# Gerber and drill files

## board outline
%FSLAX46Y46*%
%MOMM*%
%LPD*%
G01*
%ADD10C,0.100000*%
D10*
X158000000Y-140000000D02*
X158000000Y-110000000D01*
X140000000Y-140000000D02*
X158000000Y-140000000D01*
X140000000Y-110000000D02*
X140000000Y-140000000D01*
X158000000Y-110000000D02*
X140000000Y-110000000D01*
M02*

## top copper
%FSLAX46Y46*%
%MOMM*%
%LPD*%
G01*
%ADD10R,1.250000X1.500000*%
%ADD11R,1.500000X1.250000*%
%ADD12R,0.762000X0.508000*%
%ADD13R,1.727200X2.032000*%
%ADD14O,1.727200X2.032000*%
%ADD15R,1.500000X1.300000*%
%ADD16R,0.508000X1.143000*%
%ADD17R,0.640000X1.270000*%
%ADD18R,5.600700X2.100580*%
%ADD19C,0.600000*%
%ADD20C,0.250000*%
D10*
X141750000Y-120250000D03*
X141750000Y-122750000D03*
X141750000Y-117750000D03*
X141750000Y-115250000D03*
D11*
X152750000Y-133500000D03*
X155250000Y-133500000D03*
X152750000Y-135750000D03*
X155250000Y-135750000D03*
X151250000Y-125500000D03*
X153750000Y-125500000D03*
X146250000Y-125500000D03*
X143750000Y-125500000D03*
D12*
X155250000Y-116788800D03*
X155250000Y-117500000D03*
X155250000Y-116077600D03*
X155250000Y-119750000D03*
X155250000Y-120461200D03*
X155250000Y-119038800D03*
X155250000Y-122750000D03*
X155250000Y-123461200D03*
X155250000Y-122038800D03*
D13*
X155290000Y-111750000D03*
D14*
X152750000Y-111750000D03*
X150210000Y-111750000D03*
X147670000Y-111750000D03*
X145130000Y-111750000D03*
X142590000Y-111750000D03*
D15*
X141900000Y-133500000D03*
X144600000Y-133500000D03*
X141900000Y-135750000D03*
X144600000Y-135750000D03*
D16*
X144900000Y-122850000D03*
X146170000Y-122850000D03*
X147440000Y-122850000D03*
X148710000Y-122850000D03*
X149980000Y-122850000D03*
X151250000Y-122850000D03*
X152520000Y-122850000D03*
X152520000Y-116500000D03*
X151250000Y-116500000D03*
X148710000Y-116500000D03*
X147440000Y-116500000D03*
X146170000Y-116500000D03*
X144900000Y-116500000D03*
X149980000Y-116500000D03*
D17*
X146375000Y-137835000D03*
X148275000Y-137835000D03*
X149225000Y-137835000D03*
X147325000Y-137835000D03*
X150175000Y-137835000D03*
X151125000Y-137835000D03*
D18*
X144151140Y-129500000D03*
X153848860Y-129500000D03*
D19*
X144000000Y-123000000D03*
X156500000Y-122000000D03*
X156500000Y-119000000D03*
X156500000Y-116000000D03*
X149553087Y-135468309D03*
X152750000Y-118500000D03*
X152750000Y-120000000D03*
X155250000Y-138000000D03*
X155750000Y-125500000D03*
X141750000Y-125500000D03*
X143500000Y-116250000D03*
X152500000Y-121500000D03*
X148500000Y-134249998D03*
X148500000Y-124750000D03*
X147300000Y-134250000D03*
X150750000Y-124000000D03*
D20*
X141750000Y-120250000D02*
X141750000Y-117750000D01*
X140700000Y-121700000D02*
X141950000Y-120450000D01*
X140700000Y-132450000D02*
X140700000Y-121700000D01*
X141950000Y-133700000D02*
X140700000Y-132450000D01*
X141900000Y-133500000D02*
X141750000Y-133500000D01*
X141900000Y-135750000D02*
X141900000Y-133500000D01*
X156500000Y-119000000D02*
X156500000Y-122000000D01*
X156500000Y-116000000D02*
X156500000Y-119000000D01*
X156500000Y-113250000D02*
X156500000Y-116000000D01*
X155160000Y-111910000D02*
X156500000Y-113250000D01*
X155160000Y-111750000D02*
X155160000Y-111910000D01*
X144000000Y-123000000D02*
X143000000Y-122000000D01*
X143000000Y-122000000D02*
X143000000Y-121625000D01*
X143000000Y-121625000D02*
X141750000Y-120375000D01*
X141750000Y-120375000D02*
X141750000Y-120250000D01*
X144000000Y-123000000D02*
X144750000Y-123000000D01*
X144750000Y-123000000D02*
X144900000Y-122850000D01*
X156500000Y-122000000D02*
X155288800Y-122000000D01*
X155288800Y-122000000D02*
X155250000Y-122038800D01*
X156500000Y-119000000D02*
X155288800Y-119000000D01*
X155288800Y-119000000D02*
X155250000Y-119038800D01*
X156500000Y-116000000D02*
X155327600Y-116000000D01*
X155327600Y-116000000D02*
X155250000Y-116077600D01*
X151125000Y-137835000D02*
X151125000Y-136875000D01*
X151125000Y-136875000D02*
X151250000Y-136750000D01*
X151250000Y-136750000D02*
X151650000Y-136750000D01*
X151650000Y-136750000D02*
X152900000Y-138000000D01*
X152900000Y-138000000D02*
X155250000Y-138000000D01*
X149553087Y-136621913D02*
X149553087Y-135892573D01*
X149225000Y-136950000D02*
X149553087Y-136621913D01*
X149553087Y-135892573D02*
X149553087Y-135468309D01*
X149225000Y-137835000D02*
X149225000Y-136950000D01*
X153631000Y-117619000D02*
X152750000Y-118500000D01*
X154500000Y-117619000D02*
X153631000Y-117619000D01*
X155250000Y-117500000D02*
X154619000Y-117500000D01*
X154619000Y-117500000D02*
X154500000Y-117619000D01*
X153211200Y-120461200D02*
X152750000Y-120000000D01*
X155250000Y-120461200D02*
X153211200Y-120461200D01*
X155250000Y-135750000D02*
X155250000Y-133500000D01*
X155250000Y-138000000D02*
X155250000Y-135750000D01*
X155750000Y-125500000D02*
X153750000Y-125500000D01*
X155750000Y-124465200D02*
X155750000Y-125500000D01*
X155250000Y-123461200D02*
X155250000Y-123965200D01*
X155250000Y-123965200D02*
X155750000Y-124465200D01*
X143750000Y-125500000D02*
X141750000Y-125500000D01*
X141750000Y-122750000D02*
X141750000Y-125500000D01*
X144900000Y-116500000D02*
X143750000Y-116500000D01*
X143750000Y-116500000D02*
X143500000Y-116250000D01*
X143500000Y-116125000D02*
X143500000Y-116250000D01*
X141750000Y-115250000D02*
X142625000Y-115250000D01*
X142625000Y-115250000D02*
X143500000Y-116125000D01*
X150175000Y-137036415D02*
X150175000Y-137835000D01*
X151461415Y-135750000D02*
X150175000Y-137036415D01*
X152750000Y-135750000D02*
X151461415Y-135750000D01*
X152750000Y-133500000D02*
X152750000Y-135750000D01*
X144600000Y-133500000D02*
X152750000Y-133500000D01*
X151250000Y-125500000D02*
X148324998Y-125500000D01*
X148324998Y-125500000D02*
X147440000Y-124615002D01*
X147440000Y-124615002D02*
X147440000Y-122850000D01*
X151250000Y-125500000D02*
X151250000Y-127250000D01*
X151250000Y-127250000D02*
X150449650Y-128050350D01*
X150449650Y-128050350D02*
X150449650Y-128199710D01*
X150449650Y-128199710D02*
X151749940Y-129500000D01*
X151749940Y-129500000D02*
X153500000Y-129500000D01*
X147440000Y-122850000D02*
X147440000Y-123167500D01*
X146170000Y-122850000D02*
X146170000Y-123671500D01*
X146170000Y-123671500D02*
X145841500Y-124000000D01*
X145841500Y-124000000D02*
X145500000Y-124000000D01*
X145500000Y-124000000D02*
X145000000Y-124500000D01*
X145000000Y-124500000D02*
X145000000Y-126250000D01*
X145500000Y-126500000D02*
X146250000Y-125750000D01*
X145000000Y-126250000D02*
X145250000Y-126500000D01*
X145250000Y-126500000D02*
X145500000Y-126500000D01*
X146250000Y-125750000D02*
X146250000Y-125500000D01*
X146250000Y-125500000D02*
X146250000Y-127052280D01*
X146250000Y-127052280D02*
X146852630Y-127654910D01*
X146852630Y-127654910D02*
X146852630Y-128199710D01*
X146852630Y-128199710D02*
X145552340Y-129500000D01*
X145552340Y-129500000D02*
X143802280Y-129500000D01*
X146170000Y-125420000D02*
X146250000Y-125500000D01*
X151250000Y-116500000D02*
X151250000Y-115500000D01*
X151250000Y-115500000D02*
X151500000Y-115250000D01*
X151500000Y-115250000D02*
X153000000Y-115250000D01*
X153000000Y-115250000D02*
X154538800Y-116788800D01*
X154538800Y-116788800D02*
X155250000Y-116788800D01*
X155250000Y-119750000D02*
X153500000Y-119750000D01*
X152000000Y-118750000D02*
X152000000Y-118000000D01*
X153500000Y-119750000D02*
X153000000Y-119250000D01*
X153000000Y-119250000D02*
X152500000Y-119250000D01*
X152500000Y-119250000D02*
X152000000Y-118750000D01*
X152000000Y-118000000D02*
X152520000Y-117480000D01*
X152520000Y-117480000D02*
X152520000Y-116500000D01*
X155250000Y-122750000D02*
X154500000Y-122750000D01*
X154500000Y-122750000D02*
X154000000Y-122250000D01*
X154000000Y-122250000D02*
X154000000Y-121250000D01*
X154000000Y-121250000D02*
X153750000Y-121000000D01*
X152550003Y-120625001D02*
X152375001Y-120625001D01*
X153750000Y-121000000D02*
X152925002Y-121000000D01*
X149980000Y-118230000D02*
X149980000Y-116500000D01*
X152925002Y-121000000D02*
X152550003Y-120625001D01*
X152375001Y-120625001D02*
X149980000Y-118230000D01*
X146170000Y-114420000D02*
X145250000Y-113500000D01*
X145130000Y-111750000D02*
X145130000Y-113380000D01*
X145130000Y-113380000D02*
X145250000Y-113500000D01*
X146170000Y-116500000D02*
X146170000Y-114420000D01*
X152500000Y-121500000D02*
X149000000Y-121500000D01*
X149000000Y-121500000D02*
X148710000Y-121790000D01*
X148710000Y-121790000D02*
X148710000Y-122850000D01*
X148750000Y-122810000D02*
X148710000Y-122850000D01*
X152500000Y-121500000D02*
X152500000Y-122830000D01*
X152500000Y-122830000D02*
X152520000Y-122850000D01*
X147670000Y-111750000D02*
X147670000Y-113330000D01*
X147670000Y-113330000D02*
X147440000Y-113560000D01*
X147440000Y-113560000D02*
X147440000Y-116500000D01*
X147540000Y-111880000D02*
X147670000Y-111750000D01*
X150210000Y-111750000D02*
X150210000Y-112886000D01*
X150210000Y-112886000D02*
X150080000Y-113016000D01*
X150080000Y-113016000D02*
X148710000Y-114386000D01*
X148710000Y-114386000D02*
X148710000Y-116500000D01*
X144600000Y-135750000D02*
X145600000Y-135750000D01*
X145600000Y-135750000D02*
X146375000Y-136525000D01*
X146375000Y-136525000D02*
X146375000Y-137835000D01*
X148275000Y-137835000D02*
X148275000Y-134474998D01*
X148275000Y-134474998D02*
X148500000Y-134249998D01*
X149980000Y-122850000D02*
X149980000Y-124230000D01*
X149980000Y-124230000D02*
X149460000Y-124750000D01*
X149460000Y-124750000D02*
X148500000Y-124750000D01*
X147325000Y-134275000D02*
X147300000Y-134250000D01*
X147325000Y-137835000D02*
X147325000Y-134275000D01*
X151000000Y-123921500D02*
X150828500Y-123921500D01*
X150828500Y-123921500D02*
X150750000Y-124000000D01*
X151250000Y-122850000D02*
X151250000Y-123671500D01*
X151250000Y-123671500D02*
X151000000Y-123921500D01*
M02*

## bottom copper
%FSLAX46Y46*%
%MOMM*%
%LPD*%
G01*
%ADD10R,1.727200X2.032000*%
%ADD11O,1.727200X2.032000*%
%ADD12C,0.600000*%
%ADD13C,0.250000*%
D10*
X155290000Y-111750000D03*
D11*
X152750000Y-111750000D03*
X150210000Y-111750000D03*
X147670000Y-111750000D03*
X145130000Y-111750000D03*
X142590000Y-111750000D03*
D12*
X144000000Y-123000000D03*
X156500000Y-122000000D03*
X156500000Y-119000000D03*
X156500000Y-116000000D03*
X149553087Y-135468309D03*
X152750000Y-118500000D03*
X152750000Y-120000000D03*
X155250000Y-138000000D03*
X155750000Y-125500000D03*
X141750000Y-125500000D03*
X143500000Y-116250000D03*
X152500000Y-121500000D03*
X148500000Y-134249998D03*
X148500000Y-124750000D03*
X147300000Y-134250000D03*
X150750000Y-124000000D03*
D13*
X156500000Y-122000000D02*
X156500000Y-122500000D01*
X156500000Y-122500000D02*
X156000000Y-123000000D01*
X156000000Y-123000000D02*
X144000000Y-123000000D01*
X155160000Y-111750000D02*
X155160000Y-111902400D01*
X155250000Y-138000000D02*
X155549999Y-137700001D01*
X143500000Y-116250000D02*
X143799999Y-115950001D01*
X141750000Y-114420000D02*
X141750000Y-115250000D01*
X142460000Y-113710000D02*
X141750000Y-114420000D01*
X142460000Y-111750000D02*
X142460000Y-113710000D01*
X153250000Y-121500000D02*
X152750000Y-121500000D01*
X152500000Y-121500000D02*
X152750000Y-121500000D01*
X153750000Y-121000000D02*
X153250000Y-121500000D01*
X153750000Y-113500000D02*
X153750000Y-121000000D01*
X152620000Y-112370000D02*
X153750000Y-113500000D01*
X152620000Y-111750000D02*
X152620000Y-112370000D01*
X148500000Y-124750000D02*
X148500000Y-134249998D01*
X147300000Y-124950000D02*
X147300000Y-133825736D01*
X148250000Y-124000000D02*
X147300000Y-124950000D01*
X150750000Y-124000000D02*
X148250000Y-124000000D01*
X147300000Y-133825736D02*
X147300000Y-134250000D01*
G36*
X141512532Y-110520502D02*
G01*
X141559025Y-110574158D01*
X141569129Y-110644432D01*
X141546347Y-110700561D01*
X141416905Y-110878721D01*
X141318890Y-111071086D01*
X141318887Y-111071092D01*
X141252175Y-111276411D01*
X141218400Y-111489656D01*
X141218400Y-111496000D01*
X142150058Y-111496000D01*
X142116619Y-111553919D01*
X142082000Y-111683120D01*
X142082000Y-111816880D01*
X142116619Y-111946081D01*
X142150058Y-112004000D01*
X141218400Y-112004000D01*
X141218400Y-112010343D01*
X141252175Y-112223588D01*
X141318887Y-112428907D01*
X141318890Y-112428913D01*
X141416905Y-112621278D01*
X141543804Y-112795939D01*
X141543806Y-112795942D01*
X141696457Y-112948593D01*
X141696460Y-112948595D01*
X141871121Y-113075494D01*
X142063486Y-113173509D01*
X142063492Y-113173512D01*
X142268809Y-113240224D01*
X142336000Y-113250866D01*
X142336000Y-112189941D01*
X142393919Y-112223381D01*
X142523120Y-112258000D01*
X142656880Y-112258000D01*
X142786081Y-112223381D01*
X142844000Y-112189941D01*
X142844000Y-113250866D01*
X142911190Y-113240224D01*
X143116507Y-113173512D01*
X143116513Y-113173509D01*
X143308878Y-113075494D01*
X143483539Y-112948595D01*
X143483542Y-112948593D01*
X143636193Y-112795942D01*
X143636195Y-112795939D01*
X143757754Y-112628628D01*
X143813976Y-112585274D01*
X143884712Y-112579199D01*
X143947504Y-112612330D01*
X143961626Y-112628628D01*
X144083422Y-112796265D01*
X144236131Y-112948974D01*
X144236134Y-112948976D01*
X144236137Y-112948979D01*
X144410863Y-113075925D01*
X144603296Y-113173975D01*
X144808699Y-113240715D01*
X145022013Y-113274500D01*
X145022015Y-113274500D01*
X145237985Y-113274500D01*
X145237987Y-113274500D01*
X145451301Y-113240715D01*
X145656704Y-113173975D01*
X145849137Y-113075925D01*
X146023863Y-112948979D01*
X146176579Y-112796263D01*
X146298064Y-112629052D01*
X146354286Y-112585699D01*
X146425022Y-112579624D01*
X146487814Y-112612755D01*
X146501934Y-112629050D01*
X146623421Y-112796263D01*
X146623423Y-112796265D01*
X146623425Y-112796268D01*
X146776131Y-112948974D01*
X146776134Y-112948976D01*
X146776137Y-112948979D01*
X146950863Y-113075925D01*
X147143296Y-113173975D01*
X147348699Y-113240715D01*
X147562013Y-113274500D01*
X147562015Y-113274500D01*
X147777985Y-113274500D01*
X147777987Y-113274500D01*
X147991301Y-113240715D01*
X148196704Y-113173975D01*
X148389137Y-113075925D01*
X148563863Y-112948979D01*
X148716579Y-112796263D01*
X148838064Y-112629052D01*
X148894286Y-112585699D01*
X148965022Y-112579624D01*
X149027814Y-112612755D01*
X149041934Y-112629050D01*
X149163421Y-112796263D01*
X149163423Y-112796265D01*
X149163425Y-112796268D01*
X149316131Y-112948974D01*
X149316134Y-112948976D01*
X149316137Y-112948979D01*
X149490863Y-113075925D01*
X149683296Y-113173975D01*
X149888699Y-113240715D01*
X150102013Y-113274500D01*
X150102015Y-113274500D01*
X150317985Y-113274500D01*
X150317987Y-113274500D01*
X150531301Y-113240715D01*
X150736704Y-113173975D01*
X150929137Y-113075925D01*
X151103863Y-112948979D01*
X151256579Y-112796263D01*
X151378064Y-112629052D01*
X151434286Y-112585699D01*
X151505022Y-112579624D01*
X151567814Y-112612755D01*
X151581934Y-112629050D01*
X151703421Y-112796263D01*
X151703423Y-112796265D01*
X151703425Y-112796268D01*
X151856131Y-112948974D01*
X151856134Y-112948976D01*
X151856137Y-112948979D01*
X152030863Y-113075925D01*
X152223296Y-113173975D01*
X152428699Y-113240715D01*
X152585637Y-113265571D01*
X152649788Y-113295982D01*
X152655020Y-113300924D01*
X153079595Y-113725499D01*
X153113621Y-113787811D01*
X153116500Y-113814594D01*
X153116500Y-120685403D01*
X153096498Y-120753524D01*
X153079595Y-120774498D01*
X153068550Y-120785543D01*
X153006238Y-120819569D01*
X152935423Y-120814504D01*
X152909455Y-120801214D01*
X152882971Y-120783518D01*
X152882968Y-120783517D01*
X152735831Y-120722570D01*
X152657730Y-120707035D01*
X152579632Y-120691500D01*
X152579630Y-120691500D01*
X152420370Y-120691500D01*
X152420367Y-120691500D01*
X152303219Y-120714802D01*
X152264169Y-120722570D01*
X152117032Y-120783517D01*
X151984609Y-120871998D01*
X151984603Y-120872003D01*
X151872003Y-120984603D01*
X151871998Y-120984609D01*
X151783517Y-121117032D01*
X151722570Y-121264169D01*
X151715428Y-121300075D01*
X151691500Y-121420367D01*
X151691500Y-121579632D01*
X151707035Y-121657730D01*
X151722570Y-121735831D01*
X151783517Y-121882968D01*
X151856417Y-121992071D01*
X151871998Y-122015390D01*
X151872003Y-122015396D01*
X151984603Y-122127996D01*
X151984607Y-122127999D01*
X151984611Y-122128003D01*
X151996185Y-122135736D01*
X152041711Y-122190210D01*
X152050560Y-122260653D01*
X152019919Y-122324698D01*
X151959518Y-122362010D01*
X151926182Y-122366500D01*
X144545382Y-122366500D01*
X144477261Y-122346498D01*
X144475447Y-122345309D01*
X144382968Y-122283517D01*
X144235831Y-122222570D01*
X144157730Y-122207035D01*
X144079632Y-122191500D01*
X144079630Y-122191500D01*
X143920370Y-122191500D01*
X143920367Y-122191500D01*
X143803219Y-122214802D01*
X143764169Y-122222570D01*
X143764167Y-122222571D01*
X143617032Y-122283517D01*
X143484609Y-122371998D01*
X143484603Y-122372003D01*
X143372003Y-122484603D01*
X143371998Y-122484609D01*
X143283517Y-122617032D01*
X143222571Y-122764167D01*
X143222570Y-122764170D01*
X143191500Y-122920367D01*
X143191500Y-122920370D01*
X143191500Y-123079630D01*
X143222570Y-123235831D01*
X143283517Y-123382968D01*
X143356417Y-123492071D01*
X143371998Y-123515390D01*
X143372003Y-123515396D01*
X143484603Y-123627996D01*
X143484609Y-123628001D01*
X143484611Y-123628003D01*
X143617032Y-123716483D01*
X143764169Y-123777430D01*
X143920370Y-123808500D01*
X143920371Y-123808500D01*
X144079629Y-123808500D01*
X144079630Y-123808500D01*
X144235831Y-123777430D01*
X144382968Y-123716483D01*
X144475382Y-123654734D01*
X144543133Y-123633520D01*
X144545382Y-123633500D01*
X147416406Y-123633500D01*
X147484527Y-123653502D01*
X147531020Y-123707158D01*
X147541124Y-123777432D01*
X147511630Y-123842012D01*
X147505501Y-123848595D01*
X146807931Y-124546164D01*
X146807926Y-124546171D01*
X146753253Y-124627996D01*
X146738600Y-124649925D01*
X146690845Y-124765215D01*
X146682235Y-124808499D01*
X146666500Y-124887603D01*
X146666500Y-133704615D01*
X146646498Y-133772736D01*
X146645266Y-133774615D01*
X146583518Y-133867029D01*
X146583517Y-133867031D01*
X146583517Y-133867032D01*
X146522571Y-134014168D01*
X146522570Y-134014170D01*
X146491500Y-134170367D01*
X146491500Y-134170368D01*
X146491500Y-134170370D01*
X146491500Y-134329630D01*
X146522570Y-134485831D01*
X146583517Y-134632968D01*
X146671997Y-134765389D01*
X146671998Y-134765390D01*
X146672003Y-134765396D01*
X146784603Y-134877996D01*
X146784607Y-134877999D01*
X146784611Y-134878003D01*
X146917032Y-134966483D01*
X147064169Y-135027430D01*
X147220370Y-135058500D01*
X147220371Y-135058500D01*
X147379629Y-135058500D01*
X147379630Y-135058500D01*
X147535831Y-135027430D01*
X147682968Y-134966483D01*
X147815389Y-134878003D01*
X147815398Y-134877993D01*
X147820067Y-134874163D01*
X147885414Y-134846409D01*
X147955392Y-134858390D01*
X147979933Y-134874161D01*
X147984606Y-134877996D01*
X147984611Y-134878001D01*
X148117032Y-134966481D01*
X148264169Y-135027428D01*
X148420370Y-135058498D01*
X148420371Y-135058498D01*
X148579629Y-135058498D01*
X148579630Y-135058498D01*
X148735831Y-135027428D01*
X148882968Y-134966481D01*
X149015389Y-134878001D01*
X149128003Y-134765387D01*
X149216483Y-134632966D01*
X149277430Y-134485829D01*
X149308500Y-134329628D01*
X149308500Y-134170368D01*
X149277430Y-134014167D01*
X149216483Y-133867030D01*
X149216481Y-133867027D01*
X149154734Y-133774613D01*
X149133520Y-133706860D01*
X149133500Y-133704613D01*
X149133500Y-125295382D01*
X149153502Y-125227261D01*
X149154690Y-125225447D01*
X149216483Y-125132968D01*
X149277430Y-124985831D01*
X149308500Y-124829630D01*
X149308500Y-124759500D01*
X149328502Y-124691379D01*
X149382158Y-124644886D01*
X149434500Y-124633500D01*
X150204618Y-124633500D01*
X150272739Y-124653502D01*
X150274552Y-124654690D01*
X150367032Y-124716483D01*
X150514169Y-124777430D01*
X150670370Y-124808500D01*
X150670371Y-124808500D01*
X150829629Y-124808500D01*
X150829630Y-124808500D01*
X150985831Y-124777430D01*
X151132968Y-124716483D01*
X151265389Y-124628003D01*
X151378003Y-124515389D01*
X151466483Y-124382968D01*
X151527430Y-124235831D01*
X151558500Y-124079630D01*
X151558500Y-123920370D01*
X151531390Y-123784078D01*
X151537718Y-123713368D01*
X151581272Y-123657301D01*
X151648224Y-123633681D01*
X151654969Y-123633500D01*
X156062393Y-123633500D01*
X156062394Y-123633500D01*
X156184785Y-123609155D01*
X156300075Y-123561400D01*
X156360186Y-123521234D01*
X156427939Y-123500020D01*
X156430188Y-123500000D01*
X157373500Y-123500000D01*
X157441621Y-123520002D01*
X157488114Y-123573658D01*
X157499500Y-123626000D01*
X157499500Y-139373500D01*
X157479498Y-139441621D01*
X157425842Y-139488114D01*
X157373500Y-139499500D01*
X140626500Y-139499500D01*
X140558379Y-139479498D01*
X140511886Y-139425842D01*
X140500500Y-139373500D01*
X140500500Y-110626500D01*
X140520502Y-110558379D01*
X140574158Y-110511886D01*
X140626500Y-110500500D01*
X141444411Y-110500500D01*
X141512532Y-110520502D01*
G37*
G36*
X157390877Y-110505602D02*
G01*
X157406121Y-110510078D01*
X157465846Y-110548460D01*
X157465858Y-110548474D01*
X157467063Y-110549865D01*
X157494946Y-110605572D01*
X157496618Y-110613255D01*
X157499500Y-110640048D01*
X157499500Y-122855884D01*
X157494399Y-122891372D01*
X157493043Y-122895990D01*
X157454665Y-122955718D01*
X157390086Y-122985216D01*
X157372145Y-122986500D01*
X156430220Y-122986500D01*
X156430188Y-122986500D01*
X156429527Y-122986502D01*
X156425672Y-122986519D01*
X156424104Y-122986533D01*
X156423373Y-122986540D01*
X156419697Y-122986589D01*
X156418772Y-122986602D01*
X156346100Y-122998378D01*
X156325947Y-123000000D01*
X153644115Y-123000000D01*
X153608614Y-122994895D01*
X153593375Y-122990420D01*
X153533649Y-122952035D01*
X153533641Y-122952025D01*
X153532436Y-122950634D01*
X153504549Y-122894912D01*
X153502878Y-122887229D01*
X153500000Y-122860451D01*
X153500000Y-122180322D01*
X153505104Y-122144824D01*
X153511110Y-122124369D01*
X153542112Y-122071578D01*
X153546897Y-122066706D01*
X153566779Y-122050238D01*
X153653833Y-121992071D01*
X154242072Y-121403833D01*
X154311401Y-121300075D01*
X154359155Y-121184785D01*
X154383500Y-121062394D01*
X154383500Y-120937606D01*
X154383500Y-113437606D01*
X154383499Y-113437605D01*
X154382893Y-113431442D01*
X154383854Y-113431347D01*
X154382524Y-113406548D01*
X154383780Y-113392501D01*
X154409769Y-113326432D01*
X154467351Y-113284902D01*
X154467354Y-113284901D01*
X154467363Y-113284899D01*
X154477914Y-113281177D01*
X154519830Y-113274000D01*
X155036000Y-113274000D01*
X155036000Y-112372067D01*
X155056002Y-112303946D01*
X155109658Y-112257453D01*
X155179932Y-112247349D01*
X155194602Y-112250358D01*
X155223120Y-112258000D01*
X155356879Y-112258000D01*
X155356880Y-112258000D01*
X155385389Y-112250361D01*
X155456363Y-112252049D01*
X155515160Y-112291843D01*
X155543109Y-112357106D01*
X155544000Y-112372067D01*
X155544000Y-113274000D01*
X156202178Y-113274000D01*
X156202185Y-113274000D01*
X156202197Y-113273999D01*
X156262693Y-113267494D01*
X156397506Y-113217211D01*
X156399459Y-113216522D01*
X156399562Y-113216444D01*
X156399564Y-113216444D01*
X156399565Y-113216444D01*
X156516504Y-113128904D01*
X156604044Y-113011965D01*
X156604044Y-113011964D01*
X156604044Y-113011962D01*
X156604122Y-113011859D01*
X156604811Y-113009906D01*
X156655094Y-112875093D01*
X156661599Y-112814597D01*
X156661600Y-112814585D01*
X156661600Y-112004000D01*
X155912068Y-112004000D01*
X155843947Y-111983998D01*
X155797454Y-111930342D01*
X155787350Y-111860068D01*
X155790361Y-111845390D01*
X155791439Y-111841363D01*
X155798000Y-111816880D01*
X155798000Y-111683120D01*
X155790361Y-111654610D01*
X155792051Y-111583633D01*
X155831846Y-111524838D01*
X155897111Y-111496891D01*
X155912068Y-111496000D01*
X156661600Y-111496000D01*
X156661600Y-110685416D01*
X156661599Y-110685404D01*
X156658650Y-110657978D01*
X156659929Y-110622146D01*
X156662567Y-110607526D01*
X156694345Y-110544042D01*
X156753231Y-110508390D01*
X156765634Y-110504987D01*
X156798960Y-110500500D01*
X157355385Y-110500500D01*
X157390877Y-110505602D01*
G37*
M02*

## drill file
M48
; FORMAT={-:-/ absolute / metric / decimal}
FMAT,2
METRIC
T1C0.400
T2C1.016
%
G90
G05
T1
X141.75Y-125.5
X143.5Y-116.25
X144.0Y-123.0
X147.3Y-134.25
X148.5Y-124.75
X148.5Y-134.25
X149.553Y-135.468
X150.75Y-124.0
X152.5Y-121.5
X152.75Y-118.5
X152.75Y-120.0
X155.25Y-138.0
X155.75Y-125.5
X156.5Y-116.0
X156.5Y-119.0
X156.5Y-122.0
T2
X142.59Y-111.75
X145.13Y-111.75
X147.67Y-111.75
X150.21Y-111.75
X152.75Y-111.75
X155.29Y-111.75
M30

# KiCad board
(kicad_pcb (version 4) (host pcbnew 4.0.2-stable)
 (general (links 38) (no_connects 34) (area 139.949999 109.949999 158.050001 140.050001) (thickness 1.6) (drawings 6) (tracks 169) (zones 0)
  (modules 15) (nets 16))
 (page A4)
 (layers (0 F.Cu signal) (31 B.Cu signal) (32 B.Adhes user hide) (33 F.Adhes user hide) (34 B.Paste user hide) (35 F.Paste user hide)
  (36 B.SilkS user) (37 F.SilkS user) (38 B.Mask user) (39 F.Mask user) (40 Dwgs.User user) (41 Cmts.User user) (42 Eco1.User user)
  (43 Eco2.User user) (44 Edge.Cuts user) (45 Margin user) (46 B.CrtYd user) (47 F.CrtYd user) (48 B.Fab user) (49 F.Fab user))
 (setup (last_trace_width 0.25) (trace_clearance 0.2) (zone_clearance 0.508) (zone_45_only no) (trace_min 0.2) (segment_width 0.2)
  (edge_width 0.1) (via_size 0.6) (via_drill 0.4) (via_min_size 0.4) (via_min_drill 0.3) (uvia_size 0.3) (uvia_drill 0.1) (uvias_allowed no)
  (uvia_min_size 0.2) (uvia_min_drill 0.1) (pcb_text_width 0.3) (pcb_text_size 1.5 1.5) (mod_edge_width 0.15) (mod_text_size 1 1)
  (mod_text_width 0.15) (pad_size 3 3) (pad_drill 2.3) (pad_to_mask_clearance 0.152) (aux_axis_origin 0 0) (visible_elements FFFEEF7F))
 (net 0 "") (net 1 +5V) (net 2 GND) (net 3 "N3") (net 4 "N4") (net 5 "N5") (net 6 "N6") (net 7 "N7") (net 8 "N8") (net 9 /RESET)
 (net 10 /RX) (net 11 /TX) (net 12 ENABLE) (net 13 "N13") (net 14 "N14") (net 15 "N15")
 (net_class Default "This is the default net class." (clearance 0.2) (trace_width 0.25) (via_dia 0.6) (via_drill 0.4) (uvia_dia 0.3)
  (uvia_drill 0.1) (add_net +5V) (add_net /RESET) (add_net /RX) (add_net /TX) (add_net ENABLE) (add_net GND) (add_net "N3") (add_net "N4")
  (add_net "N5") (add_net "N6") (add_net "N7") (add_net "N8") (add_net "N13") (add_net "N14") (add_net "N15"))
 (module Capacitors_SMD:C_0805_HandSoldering (layer F.Cu) (at 141.75 121.5 270)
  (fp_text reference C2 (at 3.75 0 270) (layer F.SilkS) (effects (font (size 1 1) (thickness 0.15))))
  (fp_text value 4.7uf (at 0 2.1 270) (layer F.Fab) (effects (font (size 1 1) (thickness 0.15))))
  (pad 1 smd rect (at -1.25 0 270) (size 1.5 1.25) (layers F.Cu F.Paste F.Mask) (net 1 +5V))
  (pad 2 smd rect (at 1.25 0 270) (size 1.5 1.25) (layers F.Cu F.Paste F.Mask) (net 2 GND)))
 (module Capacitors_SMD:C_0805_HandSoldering (layer F.Cu) (at 141.75 116.5 90)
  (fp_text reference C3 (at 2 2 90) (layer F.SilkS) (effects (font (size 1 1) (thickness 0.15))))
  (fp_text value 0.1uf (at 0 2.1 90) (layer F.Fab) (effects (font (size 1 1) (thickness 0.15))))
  (pad 1 smd rect (at -1.25 0 90) (size 1.5 1.25) (layers F.Cu F.Paste F.Mask) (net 1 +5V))
  (pad 2 smd rect (at 1.25 0 90) (size 1.5 1.25) (layers F.Cu F.Paste F.Mask) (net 2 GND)))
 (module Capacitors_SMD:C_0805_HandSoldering (layer F.Cu) (at 154 133.5)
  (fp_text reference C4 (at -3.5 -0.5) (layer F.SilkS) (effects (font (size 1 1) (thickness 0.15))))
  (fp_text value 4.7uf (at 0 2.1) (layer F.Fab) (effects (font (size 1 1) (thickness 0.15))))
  (pad 1 smd rect (at -1.25 0) (size 1.5 1.25) (layers F.Cu F.Paste F.Mask) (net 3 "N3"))
  (pad 2 smd rect (at 1.25 0) (size 1.5 1.25) (layers F.Cu F.Paste F.Mask) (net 2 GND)))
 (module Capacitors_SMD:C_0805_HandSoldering (layer F.Cu) (at 154 135.75)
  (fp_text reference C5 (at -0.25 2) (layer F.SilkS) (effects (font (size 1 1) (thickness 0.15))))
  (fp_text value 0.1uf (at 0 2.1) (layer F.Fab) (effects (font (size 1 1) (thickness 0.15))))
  (pad 1 smd rect (at -1.25 0) (size 1.5 1.25) (layers F.Cu F.Paste F.Mask) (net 3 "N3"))
  (pad 2 smd rect (at 1.25 0) (size 1.5 1.25) (layers F.Cu F.Paste F.Mask) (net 2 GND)))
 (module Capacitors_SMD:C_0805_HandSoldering (layer F.Cu) (at 152.5 125.5)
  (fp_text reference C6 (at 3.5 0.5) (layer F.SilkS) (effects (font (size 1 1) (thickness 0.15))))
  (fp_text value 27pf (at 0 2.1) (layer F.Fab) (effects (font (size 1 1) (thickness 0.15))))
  (pad 1 smd rect (at -1.25 0) (size 1.5 1.25) (layers F.Cu F.Paste F.Mask) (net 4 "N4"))
  (pad 2 smd rect (at 1.25 0) (size 1.5 1.25) (layers F.Cu F.Paste F.Mask) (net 2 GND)))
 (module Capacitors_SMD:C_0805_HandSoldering (layer F.Cu) (at 145 125.5 180)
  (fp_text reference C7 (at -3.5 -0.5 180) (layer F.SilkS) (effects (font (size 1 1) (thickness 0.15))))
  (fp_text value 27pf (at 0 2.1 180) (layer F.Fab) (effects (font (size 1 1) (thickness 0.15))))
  (pad 1 smd rect (at -1.25 0 180) (size 1.5 1.25) (layers F.Cu F.Paste F.Mask) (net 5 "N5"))
  (pad 2 smd rect (at 1.25 0 180) (size 1.5 1.25) (layers F.Cu F.Paste F.Mask) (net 2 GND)))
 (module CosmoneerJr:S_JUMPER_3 (layer F.Cu) (at 155.25 116.7888 90)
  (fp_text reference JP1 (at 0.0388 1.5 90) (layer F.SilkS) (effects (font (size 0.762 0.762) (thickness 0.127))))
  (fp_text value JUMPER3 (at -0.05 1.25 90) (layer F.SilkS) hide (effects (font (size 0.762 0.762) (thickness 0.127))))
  (pad 2 smd rect (at 0 0 90) (size 0.508 0.762) (layers F.Cu F.Paste F.Mask) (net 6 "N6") (clearance 0.2032))
  (pad 1 smd rect (at -0.7112 0 90) (size 0.508 0.762) (layers F.Cu F.Paste F.Mask) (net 2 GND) (clearance 0.2032))
  (pad 3 smd rect (at 0.7112 0 90) (size 0.508 0.762) (layers F.Cu F.Paste F.Mask) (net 1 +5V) (clearance 0.2032)))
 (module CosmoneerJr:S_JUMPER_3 (layer F.Cu) (at 155.25 119.75 90)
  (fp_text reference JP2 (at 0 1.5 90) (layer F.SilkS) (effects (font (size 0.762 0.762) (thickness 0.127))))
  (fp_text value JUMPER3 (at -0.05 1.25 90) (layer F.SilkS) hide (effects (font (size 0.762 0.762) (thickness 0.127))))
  (pad 2 smd rect (at 0 0 90) (size 0.508 0.762) (layers F.Cu F.Paste F.Mask) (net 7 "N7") (clearance 0.2032))
  (pad 1 smd rect (at -0.7112 0 90) (size 0.508 0.762) (layers F.Cu F.Paste F.Mask) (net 2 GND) (clearance 0.2032))
  (pad 3 smd rect (at 0.7112 0 90) (size 0.508 0.762) (layers F.Cu F.Paste F.Mask) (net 1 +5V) (clearance 0.2032)))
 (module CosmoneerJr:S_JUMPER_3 (layer F.Cu) (at 155.25 122.75 90)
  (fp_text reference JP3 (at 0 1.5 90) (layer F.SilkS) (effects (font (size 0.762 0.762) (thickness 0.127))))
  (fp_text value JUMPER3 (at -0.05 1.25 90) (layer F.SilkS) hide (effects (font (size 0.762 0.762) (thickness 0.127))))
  (pad 2 smd rect (at 0 0 90) (size 0.508 0.762) (layers F.Cu F.Paste F.Mask) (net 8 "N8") (clearance 0.2032))
  (pad 1 smd rect (at -0.7112 0 90) (size 0.508 0.762) (layers F.Cu F.Paste F.Mask) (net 2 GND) (clearance 0.2032))
  (pad 3 smd rect (at 0.7112 0 90) (size 0.508 0.762) (layers F.Cu F.Paste F.Mask) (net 1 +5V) (clearance 0.2032)))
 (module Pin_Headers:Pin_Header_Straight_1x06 (layer F.Cu) (at 155.29 111.75 270)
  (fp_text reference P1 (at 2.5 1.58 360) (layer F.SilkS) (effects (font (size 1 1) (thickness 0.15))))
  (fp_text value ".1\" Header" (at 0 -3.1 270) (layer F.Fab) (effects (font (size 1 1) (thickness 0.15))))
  (pad 1 thru_hole rect (at 0 0 270) (size 2.032 1.7272) (drill 1.016) (layers *.Cu *.Mask F.SilkS) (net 1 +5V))
  (pad 2 thru_hole oval (at 0 2.54 270) (size 2.032 1.7272) (drill 1.016) (layers *.Cu *.Mask F.SilkS) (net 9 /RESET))
  (pad 3 thru_hole oval (at 0 5.08 270) (size 2.032 1.7272) (drill 1.016) (layers *.Cu *.Mask F.SilkS) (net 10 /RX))
  (pad 4 thru_hole oval (at 0 7.62 270) (size 2.032 1.7272) (drill 1.016) (layers *.Cu *.Mask F.SilkS) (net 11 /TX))
  (pad 5 thru_hole oval (at 0 10.16 270) (size 2.032 1.7272) (drill 1.016) (layers *.Cu *.Mask F.SilkS) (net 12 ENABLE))
  (pad 6 thru_hole oval (at 0 12.7 270) (size 2.032 1.7272) (drill 1.016) (layers *.Cu *.Mask F.SilkS) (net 2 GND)))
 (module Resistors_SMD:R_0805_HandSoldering (layer F.Cu) (at 143.25 133.5)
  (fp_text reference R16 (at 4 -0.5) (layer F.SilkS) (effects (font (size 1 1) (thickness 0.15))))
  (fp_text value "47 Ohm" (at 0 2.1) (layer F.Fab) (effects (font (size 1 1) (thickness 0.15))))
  (pad 1 smd rect (at -1.35 0) (size 1.5 1.3) (layers F.Cu F.Paste F.Mask) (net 1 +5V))
  (pad 2 smd rect (at 1.35 0) (size 1.5 1.3) (layers F.Cu F.Paste F.Mask) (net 3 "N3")))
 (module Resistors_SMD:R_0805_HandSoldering (layer F.Cu) (at 143.25 135.75)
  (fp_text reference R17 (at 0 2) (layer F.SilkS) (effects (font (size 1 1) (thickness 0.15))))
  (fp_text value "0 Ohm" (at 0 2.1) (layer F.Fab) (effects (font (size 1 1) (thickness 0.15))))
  (pad 1 smd rect (at -1.35 0) (size 1.5 1.3) (layers F.Cu F.Paste F.Mask) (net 1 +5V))
  (pad 2 smd rect (at 1.35 0) (size 1.5 1.3) (layers F.Cu F.Paste F.Mask) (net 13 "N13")))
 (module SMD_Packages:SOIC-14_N (layer F.Cu) (at 148.71 119.548)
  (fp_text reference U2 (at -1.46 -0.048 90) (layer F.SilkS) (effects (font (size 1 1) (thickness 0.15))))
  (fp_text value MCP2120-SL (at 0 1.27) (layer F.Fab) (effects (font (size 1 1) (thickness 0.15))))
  (pad 1 smd rect (at -3.81 3.302) (size 0.508 1.143) (layers F.Cu F.Paste F.Mask) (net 1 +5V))
  (pad 2 smd rect (at -2.54 3.302) (size 0.508 1.143) (layers F.Cu F.Paste F.Mask) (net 5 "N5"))
  (pad 3 smd rect (at -1.27 3.302) (size 0.508 1.143) (layers F.Cu F.Paste F.Mask) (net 4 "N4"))
  (pad 4 smd rect (at 0 3.302) (size 0.508 1.143) (layers F.Cu F.Paste F.Mask) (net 9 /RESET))
  (pad 5 smd rect (at 1.27 3.302) (size 0.508 1.143) (layers F.Cu F.Paste F.Mask) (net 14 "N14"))
  (pad 6 smd rect (at 2.54 3.302) (size 0.508 1.143) (layers F.Cu F.Paste F.Mask) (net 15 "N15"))
  (pad 7 smd rect (at 3.81 3.302) (size 0.508 1.143) (layers F.Cu F.Paste F.Mask) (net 9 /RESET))
  (pad 8 smd rect (at 3.81 -3.048) (size 0.508 1.143) (layers F.Cu F.Paste F.Mask) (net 7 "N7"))
  (pad 9 smd rect (at 2.54 -3.048) (size 0.508 1.143) (layers F.Cu F.Paste F.Mask) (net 6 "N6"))
  (pad 11 smd rect (at 0 -3.048) (size 0.508 1.143) (layers F.Cu F.Paste F.Mask) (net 10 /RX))
  (pad 12 smd rect (at -1.27 -3.048) (size 0.508 1.143) (layers F.Cu F.Paste F.Mask) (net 11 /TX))
  (pad 13 smd rect (at -2.54 -3.048) (size 0.508 1.143) (layers F.Cu F.Paste F.Mask) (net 12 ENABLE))
  (pad 14 smd rect (at -3.81 -3.048) (size 0.508 1.143) (layers F.Cu F.Paste F.Mask) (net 2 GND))
  (pad 10 smd rect (at 1.27 -3.048) (size 0.508 1.143) (layers F.Cu F.Paste F.Mask) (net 8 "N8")))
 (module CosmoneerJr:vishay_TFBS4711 (layer F.Cu) (at 148.75 138.5)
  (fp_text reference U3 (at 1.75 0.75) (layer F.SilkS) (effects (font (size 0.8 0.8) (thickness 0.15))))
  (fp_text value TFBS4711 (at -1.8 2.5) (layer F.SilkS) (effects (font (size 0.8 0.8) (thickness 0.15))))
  (pad 1 smd rect (at -2.375 -0.665) (size 0.64 1.27) (layers F.Cu F.Paste F.Mask) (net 13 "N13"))
  (pad 3 smd rect (at -0.475 -0.665) (size 0.64 1.27) (layers F.Cu F.Paste F.Mask) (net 14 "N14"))
  (pad 4 smd rect (at 0.475 -0.665) (size 0.64 1.27) (layers F.Cu F.Paste F.Mask) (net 2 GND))
  (pad 2 smd rect (at -1.425 -0.665) (size 0.64 1.27) (layers F.Cu F.Paste F.Mask) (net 15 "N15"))
  (pad 5 smd rect (at 1.425 -0.665) (size 0.64 1.27) (layers F.Cu F.Paste F.Mask) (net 3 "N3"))
  (pad 6 smd rect (at 2.375 -0.665) (size 0.64 1.27) (layers F.Cu F.Paste F.Mask) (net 2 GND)))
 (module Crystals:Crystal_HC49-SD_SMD (layer F.Cu) (at 149 129.5)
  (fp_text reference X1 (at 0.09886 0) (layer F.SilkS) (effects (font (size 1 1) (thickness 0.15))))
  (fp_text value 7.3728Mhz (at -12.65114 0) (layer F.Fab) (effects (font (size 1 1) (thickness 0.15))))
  (pad 1 smd rect (at -4.84886 0) (size 5.6007 2.10058) (layers F.Cu F.Paste F.Mask) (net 5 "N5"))
  (pad 2 smd rect (at 4.84886 0) (size 5.6007 2.10058) (layers F.Cu F.Paste F.Mask) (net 4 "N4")))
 (gr_line (start 158 140) (end 158 110) (layer Edge.Cuts) (width 0.1))
 (gr_line (start 140 140) (end 158 140) (layer Edge.Cuts) (width 0.1))
 (gr_line (start 140 110) (end 140 140) (layer Edge.Cuts) (width 0.1))
 (gr_line (start 158 110) (end 140 110) (layer Edge.Cuts) (width 0.1))
 (segment (start 141.75 120.25) (end 141.75 117.75) (width 0.25) (layer F.Cu) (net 1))
 (segment (start 140.7 121.7) (end 141.95 120.45) (width 0.25) (layer F.Cu) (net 1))
 (segment (start 140.7 132.45) (end 140.7 121.7) (width 0.25) (layer F.Cu) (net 1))
 (segment (start 141.95 133.7) (end 140.7 132.45) (width 0.25) (layer F.Cu) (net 1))
 (segment (start 141.9 133.5) (end 141.75 133.5) (width 0.25) (layer F.Cu) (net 1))
 (segment (start 141.9 135.75) (end 141.9 133.5) (width 0.25) (layer F.Cu) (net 1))
 (segment (start 156.5 119) (end 156.5 122) (width 0.25) (layer F.Cu) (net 1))
 (segment (start 156.5 116) (end 156.5 119) (width 0.25) (layer F.Cu) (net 1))
 (segment (start 156.5 113.25) (end 156.5 116) (width 0.25) (layer F.Cu) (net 1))
 (segment (start 155.16 111.91) (end 156.5 113.25) (width 0.25) (layer F.Cu) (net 1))
 (segment (start 155.16 111.75) (end 155.16 111.91) (width 0.25) (layer F.Cu) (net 1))
 (segment (start 144 123) (end 143 122) (width 0.25) (layer F.Cu) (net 1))
 (segment (start 143 122) (end 143 121.625) (width 0.25) (layer F.Cu) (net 1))
 (segment (start 143 121.625) (end 141.75 120.375) (width 0.25) (layer F.Cu) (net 1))
 (segment (start 141.75 120.375) (end 141.75 120.25) (width 0.25) (layer F.Cu) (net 1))
 (segment (start 144 123) (end 144.75 123) (width 0.25) (layer F.Cu) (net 1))
 (segment (start 144.75 123) (end 144.9 122.85) (width 0.25) (layer F.Cu) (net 1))
 (via (at 144 123) (size 0.6) (drill 0.4) (layers F.Cu B.Cu) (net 1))
 (segment (start 156.5 122) (end 156.5 122.5) (width 0.25) (layer B.Cu) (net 1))
 (segment (start 156.5 122.5) (end 156 123) (width 0.25) (layer B.Cu) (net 1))
 (segment (start 156 123) (end 144 123) (width 0.25) (layer B.Cu) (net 1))
 (segment (start 156.5 122) (end 155.2888 122) (width 0.25) (layer F.Cu) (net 1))
 (segment (start 155.2888 122) (end 155.25 122.0388) (width 0.25) (layer F.Cu) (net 1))
 (segment (start 156.5 119) (end 155.2888 119) (width 0.25) (layer F.Cu) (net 1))
 (segment (start 155.2888 119) (end 155.25 119.0388) (width 0.25) (layer F.Cu) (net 1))
 (via (at 156.5 122) (size 0.6) (drill 0.4) (layers F.Cu B.Cu) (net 1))
 (via (at 156.5 119) (size 0.6) (drill 0.4) (layers F.Cu B.Cu) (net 1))
 (segment (start 156.5 116) (end 155.3276 116) (width 0.25) (layer F.Cu) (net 1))
 (segment (start 155.3276 116) (end 155.25 116.0776) (width 0.25) (layer F.Cu) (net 1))
 (via (at 156.5 116) (size 0.6) (drill 0.4) (layers F.Cu B.Cu) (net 1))
 (segment (start 155.16 111.75) (end 155.16 111.9024) (width 0.25) (layer B.Cu) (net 1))
 (segment (start 151.125 137.835) (end 151.125 136.875) (width 0.25) (layer F.Cu) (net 2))
 (segment (start 151.125 136.875) (end 151.25 136.75) (width 0.25) (layer F.Cu) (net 2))
 (segment (start 151.25 136.75) (end 151.65 136.75) (width 0.25) (layer F.Cu) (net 2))
 (segment (start 151.65 136.75) (end 152.9 138) (width 0.25) (layer F.Cu) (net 2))
 (segment (start 152.9 138) (end 155.25 138) (width 0.25) (layer F.Cu) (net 2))
 (segment (start 149.553087 136.621913) (end 149.553087 135.892573) (width 0.25) (layer F.Cu) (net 2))
 (segment (start 149.225 136.95) (end 149.553087 136.621913) (width 0.25) (layer F.Cu) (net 2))
 (segment (start 149.553087 135.892573) (end 149.553087 135.468309) (width 0.25) (layer F.Cu) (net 2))
 (via (at 149.553087 135.468309) (size 0.6) (drill 0.4) (layers F.Cu B.Cu) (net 2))
 (segment (start 149.225 137.835) (end 149.225 136.95) (width 0.25) (layer F.Cu) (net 2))
 (via (at 152.75 118.5) (size 0.6) (drill 0.4) (layers F.Cu B.Cu) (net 2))
 (segment (start 153.631 117.619) (end 152.75 118.5) (width 0.25) (layer F.Cu) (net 2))
 (segment (start 154.5 117.619) (end 153.631 117.619) (width 0.25) (layer F.Cu) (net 2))
 (segment (start 155.25 117.5) (end 154.619 117.5) (width 0.25) (layer F.Cu) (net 2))
 (segment (start 154.619 117.5) (end 154.5 117.619) (width 0.25) (layer F.Cu) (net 2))
 (via (at 152.75 120) (size 0.6) (drill 0.4) (layers F.Cu B.Cu) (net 2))
 (segment (start 153.2112 120.4612) (end 152.75 120) (width 0.25) (layer F.Cu) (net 2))
 (segment (start 155.25 120.4612) (end 153.2112 120.4612) (width 0.25) (layer F.Cu) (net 2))
 (segment (start 155.25 135.75) (end 155.25 133.5) (width 0.25) (layer F.Cu) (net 2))
 (segment (start 155.25 138) (end 155.25 135.75) (width 0.25) (layer F.Cu) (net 2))
 (segment (start 155.25 138) (end 155.549999 137.700001) (width 0.25) (layer B.Cu) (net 2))
 (via (at 155.25 138) (size 0.6) (drill 0.4) (layers F.Cu B.Cu) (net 2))
 (segment (start 155.75 125.5) (end 153.75 125.5) (width 0.25) (layer F.Cu) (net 2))
 (via (at 155.75 125.5) (size 0.6) (drill 0.4) (layers F.Cu B.Cu) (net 2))
 (segment (start 155.75 124.4652) (end 155.75 125.5) (width 0.25) (layer F.Cu) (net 2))
 (segment (start 155.25 123.4612) (end 155.25 123.9652) (width 0.25) (layer F.Cu) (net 2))
 (segment (start 155.25 123.9652) (end 155.75 124.4652) (width 0.25) (layer F.Cu) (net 2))
 (segment (start 143.75 125.5) (end 141.75 125.5) (width 0.25) (layer F.Cu) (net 2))
 (via (at 141.75 125.5) (size 0.6) (drill 0.4) (layers F.Cu B.Cu) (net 2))
 (segment (start 141.75 122.75) (end 141.75 125.5) (width 0.25) (layer F.Cu) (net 2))
 (segment (start 144.9 116.5) (end 143.75 116.5) (width 0.25) (layer F.Cu) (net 2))
 (segment (start 143.75 116.5) (end 143.5 116.25) (width 0.25) (layer F.Cu) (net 2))
 (segment (start 143.5 116.25) (end 143.799999 115.950001) (width 0.25) (layer B.Cu) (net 2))
 (segment (start 143.5 116.125) (end 143.5 116.25) (width 0.25) (layer F.Cu) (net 2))
 (via (at 143.5 116.25) (size 0.6) (drill 0.4) (layers F.Cu B.Cu) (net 2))
 (segment (start 141.75 115.25) (end 142.625 115.25) (width 0.25) (layer F.Cu) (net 2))
 (segment (start 142.625 115.25) (end 143.5 116.125) (width 0.25) (layer F.Cu) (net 2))
 (segment (start 141.75 114.42) (end 141.75 115.25) (width 0.25) (layer B.Cu) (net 2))
 (segment (start 142.46 113.71) (end 141.75 114.42) (width 0.25) (layer B.Cu) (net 2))
 (segment (start 142.46 111.75) (end 142.46 113.71) (width 0.25) (layer B.Cu) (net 2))
 (segment (start 150.175 137.036415) (end 150.175 137.835) (width 0.25) (layer F.Cu) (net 3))
 (segment (start 151.461415 135.75) (end 150.175 137.036415) (width 0.25) (layer F.Cu) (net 3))
 (segment (start 152.75 135.75) (end 151.461415 135.75) (width 0.25) (layer F.Cu) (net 3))
 (segment (start 152.75 133.5) (end 152.75 135.75) (width 0.25) (layer F.Cu) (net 3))
 (segment (start 144.6 133.5) (end 152.75 133.5) (width 0.25) (layer F.Cu) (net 3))
 (segment (start 151.25 125.5) (end 148.324998 125.5) (width 0.25) (layer F.Cu) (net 4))
 (segment (start 148.324998 125.5) (end 147.44 124.615002) (width 0.25) (layer F.Cu) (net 4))
 (segment (start 147.44 124.615002) (end 147.44 122.85) (width 0.25) (layer F.Cu) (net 4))
 (segment (start 151.25 125.5) (end 151.25 127.25) (width 0.25) (layer F.Cu) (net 4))
 (segment (start 151.25 127.25) (end 150.44965 128.05035) (width 0.25) (layer F.Cu) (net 4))
 (segment (start 150.44965 128.05035) (end 150.44965 128.19971) (width 0.25) (layer F.Cu) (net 4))
 (segment (start 150.44965 128.19971) (end 151.74994 129.5) (width 0.25) (layer F.Cu) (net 4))
 (segment (start 151.74994 129.5) (end 153.5 129.5) (width 0.25) (layer F.Cu) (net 4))
 (segment (start 147.44 122.85) (end 147.44 123.1675) (width 0.25) (layer F.Cu) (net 4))
 (segment (start 146.17 122.85) (end 146.17 123.6715) (width 0.25) (layer F.Cu) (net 5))
 (segment (start 146.17 123.6715) (end 145.8415 124) (width 0.25) (layer F.Cu) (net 5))
 (segment (start 145.8415 124) (end 145.5 124) (width 0.25) (layer F.Cu) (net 5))
 (segment (start 145.5 124) (end 145 124.5) (width 0.25) (layer F.Cu) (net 5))
 (segment (start 145 124.5) (end 145 126.25) (width 0.25) (layer F.Cu) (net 5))
 (segment (start 145.5 126.5) (end 146.25 125.75) (width 0.25) (layer F.Cu) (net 5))
 (segment (start 145 126.25) (end 145.25 126.5) (width 0.25) (layer F.Cu) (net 5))
 (segment (start 145.25 126.5) (end 145.5 126.5) (width 0.25) (layer F.Cu) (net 5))
 (segment (start 146.25 125.75) (end 146.25 125.5) (width 0.25) (layer F.Cu) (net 5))
 (segment (start 146.25 125.5) (end 146.25 127.05228) (width 0.25) (layer F.Cu) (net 5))
 (segment (start 146.25 127.05228) (end 146.85263 127.65491) (width 0.25) (layer F.Cu) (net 5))
 (segment (start 146.85263 127.65491) (end 146.85263 128.19971) (width 0.25) (layer F.Cu) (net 5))
 (segment (start 146.85263 128.19971) (end 145.55234 129.5) (width 0.25) (layer F.Cu) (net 5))
 (segment (start 145.55234 129.5) (end 143.80228 129.5) (width 0.25) (layer F.Cu) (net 5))
 (segment (start 146.17 125.42) (end 146.25 125.5) (width 0.25) (layer F.Cu) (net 5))
 (segment (start 151.25 116.5) (end 151.25 115.5) (width 0.25) (layer F.Cu) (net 6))
 (segment (start 151.25 115.5) (end 151.5 115.25) (width 0.25) (layer F.Cu) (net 6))
 (segment (start 151.5 115.25) (end 153 115.25) (width 0.25) (layer F.Cu) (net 6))
 (segment (start 153 115.25) (end 154.5388 116.7888) (width 0.25) (layer F.Cu) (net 6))
 (segment (start 154.5388 116.7888) (end 155.25 116.7888) (width 0.25) (layer F.Cu) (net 6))
 (segment (start 155.25 119.75) (end 153.5 119.75) (width 0.25) (layer F.Cu) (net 7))
 (segment (start 152 118.75) (end 152 118) (width 0.25) (layer F.Cu) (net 7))
 (segment (start 153.5 119.75) (end 153 119.25) (width 0.25) (layer F.Cu) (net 7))
 (segment (start 153 119.25) (end 152.5 119.25) (width 0.25) (layer F.Cu) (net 7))
 (segment (start 152.5 119.25) (end 152 118.75) (width 0.25) (layer F.Cu) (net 7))
 (segment (start 152 118) (end 152.52 117.48) (width 0.25) (layer F.Cu) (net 7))
 (segment (start 152.52 117.48) (end 152.52 116.5) (width 0.25) (layer F.Cu) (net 7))
 (segment (start 155.25 122.75) (end 154.5 122.75) (width 0.25) (layer F.Cu) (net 8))
 (segment (start 154.5 122.75) (end 154 122.25) (width 0.25) (layer F.Cu) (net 8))
 (segment (start 154 122.25) (end 154 121.25) (width 0.25) (layer F.Cu) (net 8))
 (segment (start 154 121.25) (end 153.75 121) (width 0.25) (layer F.Cu) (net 8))
 (segment (start 152.550003 120.625001) (end 152.375001 120.625001) (width 0.25) (layer F.Cu) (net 8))
 (segment (start 153.75 121) (end 152.925002 121) (width 0.25) (layer F.Cu) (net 8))
 (segment (start 149.98 118.23) (end 149.98 116.5) (width 0.25) (layer F.Cu) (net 8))
 (segment (start 152.925002 121) (end 152.550003 120.625001) (width 0.25) (layer F.Cu) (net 8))
 (segment (start 152.375001 120.625001) (end 149.98 118.23) (width 0.25) (layer F.Cu) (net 8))
 (segment (start 146.17 114.42) (end 145.25 113.5) (width 0.25) (layer F.Cu) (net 12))
 (segment (start 145.13 111.75) (end 145.13 113.38) (width 0.25) (layer F.Cu) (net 12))
 (segment (start 145.13 113.38) (end 145.25 113.5) (width 0.25) (layer F.Cu) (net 12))
 (segment (start 146.17 116.5) (end 146.17 114.42) (width 0.25) (layer F.Cu) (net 12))
 (segment (start 152.5 121.5) (end 149 121.5) (width 0.25) (layer F.Cu) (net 9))
 (segment (start 149 121.5) (end 148.71 121.79) (width 0.25) (layer F.Cu) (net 9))
 (segment (start 148.71 121.79) (end 148.71 122.85) (width 0.25) (layer F.Cu) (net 9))
 (segment (start 148.75 122.81) (end 148.71 122.85) (width 0.25) (layer F.Cu) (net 9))
 (segment (start 152.5 121.5) (end 152.5 122.83) (width 0.25) (layer F.Cu) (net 9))
 (segment (start 152.5 122.83) (end 152.52 122.85) (width 0.25) (layer F.Cu) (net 9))
 (via (at 152.5 121.5) (size 0.6) (drill 0.4) (layers F.Cu B.Cu) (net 9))
 (segment (start 153.25 121.5) (end 152.75 121.5) (width 0.25) (layer B.Cu) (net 9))
 (segment (start 152.5 121.5) (end 152.75 121.5) (width 0.25) (layer B.Cu) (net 9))
 (segment (start 153.75 121) (end 153.25 121.5) (width 0.25) (layer B.Cu) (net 9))
 (segment (start 153.75 113.5) (end 153.75 121) (width 0.25) (layer B.Cu) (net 9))
 (segment (start 152.62 112.37) (end 153.75 113.5) (width 0.25) (layer B.Cu) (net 9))
 (segment (start 152.62 111.75) (end 152.62 112.37) (width 0.25) (layer B.Cu) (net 9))
 (segment (start 147.67 111.75) (end 147.67 113.33) (width 0.25) (layer F.Cu) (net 11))
 (segment (start 147.67 113.33) (end 147.44 113.56) (width 0.25) (layer F.Cu) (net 11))
 (segment (start 147.44 113.56) (end 147.44 116.5) (width 0.25) (layer F.Cu) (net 11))
 (segment (start 147.54 111.88) (end 147.67 111.75) (width 0.25) (layer F.Cu) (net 11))
 (segment (start 150.21 111.75) (end 150.21 112.886) (width 0.25) (layer F.Cu) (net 10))
 (segment (start 150.21 112.886) (end 150.08 113.016) (width 0.25) (layer F.Cu) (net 10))
 (segment (start 150.08 113.016) (end 148.71 114.386) (width 0.25) (layer F.Cu) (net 10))
 (segment (start 148.71 114.386) (end 148.71 116.5) (width 0.25) (layer F.Cu) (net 10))
 (segment (start 144.6 135.75) (end 145.6 135.75) (width 0.25) (layer F.Cu) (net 13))
 (segment (start 145.6 135.75) (end 146.375 136.525) (width 0.25) (layer F.Cu) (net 13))
 (segment (start 146.375 136.525) (end 146.375 137.835) (width 0.25) (layer F.Cu) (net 13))
 (segment (start 148.275 137.835) (end 148.275 134.474998) (width 0.25) (layer F.Cu) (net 14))
 (segment (start 148.5 124.75) (end 148.5 134.249998) (width 0.25) (layer B.Cu) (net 14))
 (via (at 148.5 134.249998) (size 0.6) (drill 0.4) (layers F.Cu B.Cu) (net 14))
 (segment (start 148.275 134.474998) (end 148.5 134.249998) (width 0.25) (layer F.Cu) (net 14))
 (segment (start 149.98 122.85) (end 149.98 124.23) (width 0.25) (layer F.Cu) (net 14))
 (segment (start 149.98 124.23) (end 149.46 124.75) (width 0.25) (layer F.Cu) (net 14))
 (segment (start 149.46 124.75) (end 148.5 124.75) (width 0.25) (layer F.Cu) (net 14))
 (via (at 148.5 124.75) (size 0.6) (drill 0.4) (layers F.Cu B.Cu) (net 14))
 (segment (start 147.3 124.95) (end 147.3 133.825736) (width 0.25) (layer B.Cu) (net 15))
 (segment (start 148.25 124) (end 147.3 124.95) (width 0.25) (layer B.Cu) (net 15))
 (segment (start 150.75 124) (end 148.25 124) (width 0.25) (layer B.Cu) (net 15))
 (segment (start 147.325 134.275) (end 147.3 134.25) (width 0.25) (layer F.Cu) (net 15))
 (via (at 147.3 134.25) (size 0.6) (drill 0.4) (layers F.Cu B.Cu) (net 15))
 (segment (start 147.325 137.835) (end 147.325 134.275) (width 0.25) (layer F.Cu) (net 15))
 (segment (start 147.3 133.825736) (end 147.3 134.25) (width 0.25) (layer B.Cu) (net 15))
 (segment (start 151 123.9215) (end 150.8285 123.9215) (width 0.25) (layer F.Cu) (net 15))
 (segment (start 150.8285 123.9215) (end 150.75 124) (width 0.25) (layer F.Cu) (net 15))
 (via (at 150.75 124) (size 0.6) (drill 0.4) (layers F.Cu B.Cu) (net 15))
 (segment (start 151.25 122.85) (end 151.25 123.6715) (width 0.25) (layer F.Cu) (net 15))
 (segment (start 151.25 123.6715) (end 151 123.9215) (width 0.25) (layer F.Cu) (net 15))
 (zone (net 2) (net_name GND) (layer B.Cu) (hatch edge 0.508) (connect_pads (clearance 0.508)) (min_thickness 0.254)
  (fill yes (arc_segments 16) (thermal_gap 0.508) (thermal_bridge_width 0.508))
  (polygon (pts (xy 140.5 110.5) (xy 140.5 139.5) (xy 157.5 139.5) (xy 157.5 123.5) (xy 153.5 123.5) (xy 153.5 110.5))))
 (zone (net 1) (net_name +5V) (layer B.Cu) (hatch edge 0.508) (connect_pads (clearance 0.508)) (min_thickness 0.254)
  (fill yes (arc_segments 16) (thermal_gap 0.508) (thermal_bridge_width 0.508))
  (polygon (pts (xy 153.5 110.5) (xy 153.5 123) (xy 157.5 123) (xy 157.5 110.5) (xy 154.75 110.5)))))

